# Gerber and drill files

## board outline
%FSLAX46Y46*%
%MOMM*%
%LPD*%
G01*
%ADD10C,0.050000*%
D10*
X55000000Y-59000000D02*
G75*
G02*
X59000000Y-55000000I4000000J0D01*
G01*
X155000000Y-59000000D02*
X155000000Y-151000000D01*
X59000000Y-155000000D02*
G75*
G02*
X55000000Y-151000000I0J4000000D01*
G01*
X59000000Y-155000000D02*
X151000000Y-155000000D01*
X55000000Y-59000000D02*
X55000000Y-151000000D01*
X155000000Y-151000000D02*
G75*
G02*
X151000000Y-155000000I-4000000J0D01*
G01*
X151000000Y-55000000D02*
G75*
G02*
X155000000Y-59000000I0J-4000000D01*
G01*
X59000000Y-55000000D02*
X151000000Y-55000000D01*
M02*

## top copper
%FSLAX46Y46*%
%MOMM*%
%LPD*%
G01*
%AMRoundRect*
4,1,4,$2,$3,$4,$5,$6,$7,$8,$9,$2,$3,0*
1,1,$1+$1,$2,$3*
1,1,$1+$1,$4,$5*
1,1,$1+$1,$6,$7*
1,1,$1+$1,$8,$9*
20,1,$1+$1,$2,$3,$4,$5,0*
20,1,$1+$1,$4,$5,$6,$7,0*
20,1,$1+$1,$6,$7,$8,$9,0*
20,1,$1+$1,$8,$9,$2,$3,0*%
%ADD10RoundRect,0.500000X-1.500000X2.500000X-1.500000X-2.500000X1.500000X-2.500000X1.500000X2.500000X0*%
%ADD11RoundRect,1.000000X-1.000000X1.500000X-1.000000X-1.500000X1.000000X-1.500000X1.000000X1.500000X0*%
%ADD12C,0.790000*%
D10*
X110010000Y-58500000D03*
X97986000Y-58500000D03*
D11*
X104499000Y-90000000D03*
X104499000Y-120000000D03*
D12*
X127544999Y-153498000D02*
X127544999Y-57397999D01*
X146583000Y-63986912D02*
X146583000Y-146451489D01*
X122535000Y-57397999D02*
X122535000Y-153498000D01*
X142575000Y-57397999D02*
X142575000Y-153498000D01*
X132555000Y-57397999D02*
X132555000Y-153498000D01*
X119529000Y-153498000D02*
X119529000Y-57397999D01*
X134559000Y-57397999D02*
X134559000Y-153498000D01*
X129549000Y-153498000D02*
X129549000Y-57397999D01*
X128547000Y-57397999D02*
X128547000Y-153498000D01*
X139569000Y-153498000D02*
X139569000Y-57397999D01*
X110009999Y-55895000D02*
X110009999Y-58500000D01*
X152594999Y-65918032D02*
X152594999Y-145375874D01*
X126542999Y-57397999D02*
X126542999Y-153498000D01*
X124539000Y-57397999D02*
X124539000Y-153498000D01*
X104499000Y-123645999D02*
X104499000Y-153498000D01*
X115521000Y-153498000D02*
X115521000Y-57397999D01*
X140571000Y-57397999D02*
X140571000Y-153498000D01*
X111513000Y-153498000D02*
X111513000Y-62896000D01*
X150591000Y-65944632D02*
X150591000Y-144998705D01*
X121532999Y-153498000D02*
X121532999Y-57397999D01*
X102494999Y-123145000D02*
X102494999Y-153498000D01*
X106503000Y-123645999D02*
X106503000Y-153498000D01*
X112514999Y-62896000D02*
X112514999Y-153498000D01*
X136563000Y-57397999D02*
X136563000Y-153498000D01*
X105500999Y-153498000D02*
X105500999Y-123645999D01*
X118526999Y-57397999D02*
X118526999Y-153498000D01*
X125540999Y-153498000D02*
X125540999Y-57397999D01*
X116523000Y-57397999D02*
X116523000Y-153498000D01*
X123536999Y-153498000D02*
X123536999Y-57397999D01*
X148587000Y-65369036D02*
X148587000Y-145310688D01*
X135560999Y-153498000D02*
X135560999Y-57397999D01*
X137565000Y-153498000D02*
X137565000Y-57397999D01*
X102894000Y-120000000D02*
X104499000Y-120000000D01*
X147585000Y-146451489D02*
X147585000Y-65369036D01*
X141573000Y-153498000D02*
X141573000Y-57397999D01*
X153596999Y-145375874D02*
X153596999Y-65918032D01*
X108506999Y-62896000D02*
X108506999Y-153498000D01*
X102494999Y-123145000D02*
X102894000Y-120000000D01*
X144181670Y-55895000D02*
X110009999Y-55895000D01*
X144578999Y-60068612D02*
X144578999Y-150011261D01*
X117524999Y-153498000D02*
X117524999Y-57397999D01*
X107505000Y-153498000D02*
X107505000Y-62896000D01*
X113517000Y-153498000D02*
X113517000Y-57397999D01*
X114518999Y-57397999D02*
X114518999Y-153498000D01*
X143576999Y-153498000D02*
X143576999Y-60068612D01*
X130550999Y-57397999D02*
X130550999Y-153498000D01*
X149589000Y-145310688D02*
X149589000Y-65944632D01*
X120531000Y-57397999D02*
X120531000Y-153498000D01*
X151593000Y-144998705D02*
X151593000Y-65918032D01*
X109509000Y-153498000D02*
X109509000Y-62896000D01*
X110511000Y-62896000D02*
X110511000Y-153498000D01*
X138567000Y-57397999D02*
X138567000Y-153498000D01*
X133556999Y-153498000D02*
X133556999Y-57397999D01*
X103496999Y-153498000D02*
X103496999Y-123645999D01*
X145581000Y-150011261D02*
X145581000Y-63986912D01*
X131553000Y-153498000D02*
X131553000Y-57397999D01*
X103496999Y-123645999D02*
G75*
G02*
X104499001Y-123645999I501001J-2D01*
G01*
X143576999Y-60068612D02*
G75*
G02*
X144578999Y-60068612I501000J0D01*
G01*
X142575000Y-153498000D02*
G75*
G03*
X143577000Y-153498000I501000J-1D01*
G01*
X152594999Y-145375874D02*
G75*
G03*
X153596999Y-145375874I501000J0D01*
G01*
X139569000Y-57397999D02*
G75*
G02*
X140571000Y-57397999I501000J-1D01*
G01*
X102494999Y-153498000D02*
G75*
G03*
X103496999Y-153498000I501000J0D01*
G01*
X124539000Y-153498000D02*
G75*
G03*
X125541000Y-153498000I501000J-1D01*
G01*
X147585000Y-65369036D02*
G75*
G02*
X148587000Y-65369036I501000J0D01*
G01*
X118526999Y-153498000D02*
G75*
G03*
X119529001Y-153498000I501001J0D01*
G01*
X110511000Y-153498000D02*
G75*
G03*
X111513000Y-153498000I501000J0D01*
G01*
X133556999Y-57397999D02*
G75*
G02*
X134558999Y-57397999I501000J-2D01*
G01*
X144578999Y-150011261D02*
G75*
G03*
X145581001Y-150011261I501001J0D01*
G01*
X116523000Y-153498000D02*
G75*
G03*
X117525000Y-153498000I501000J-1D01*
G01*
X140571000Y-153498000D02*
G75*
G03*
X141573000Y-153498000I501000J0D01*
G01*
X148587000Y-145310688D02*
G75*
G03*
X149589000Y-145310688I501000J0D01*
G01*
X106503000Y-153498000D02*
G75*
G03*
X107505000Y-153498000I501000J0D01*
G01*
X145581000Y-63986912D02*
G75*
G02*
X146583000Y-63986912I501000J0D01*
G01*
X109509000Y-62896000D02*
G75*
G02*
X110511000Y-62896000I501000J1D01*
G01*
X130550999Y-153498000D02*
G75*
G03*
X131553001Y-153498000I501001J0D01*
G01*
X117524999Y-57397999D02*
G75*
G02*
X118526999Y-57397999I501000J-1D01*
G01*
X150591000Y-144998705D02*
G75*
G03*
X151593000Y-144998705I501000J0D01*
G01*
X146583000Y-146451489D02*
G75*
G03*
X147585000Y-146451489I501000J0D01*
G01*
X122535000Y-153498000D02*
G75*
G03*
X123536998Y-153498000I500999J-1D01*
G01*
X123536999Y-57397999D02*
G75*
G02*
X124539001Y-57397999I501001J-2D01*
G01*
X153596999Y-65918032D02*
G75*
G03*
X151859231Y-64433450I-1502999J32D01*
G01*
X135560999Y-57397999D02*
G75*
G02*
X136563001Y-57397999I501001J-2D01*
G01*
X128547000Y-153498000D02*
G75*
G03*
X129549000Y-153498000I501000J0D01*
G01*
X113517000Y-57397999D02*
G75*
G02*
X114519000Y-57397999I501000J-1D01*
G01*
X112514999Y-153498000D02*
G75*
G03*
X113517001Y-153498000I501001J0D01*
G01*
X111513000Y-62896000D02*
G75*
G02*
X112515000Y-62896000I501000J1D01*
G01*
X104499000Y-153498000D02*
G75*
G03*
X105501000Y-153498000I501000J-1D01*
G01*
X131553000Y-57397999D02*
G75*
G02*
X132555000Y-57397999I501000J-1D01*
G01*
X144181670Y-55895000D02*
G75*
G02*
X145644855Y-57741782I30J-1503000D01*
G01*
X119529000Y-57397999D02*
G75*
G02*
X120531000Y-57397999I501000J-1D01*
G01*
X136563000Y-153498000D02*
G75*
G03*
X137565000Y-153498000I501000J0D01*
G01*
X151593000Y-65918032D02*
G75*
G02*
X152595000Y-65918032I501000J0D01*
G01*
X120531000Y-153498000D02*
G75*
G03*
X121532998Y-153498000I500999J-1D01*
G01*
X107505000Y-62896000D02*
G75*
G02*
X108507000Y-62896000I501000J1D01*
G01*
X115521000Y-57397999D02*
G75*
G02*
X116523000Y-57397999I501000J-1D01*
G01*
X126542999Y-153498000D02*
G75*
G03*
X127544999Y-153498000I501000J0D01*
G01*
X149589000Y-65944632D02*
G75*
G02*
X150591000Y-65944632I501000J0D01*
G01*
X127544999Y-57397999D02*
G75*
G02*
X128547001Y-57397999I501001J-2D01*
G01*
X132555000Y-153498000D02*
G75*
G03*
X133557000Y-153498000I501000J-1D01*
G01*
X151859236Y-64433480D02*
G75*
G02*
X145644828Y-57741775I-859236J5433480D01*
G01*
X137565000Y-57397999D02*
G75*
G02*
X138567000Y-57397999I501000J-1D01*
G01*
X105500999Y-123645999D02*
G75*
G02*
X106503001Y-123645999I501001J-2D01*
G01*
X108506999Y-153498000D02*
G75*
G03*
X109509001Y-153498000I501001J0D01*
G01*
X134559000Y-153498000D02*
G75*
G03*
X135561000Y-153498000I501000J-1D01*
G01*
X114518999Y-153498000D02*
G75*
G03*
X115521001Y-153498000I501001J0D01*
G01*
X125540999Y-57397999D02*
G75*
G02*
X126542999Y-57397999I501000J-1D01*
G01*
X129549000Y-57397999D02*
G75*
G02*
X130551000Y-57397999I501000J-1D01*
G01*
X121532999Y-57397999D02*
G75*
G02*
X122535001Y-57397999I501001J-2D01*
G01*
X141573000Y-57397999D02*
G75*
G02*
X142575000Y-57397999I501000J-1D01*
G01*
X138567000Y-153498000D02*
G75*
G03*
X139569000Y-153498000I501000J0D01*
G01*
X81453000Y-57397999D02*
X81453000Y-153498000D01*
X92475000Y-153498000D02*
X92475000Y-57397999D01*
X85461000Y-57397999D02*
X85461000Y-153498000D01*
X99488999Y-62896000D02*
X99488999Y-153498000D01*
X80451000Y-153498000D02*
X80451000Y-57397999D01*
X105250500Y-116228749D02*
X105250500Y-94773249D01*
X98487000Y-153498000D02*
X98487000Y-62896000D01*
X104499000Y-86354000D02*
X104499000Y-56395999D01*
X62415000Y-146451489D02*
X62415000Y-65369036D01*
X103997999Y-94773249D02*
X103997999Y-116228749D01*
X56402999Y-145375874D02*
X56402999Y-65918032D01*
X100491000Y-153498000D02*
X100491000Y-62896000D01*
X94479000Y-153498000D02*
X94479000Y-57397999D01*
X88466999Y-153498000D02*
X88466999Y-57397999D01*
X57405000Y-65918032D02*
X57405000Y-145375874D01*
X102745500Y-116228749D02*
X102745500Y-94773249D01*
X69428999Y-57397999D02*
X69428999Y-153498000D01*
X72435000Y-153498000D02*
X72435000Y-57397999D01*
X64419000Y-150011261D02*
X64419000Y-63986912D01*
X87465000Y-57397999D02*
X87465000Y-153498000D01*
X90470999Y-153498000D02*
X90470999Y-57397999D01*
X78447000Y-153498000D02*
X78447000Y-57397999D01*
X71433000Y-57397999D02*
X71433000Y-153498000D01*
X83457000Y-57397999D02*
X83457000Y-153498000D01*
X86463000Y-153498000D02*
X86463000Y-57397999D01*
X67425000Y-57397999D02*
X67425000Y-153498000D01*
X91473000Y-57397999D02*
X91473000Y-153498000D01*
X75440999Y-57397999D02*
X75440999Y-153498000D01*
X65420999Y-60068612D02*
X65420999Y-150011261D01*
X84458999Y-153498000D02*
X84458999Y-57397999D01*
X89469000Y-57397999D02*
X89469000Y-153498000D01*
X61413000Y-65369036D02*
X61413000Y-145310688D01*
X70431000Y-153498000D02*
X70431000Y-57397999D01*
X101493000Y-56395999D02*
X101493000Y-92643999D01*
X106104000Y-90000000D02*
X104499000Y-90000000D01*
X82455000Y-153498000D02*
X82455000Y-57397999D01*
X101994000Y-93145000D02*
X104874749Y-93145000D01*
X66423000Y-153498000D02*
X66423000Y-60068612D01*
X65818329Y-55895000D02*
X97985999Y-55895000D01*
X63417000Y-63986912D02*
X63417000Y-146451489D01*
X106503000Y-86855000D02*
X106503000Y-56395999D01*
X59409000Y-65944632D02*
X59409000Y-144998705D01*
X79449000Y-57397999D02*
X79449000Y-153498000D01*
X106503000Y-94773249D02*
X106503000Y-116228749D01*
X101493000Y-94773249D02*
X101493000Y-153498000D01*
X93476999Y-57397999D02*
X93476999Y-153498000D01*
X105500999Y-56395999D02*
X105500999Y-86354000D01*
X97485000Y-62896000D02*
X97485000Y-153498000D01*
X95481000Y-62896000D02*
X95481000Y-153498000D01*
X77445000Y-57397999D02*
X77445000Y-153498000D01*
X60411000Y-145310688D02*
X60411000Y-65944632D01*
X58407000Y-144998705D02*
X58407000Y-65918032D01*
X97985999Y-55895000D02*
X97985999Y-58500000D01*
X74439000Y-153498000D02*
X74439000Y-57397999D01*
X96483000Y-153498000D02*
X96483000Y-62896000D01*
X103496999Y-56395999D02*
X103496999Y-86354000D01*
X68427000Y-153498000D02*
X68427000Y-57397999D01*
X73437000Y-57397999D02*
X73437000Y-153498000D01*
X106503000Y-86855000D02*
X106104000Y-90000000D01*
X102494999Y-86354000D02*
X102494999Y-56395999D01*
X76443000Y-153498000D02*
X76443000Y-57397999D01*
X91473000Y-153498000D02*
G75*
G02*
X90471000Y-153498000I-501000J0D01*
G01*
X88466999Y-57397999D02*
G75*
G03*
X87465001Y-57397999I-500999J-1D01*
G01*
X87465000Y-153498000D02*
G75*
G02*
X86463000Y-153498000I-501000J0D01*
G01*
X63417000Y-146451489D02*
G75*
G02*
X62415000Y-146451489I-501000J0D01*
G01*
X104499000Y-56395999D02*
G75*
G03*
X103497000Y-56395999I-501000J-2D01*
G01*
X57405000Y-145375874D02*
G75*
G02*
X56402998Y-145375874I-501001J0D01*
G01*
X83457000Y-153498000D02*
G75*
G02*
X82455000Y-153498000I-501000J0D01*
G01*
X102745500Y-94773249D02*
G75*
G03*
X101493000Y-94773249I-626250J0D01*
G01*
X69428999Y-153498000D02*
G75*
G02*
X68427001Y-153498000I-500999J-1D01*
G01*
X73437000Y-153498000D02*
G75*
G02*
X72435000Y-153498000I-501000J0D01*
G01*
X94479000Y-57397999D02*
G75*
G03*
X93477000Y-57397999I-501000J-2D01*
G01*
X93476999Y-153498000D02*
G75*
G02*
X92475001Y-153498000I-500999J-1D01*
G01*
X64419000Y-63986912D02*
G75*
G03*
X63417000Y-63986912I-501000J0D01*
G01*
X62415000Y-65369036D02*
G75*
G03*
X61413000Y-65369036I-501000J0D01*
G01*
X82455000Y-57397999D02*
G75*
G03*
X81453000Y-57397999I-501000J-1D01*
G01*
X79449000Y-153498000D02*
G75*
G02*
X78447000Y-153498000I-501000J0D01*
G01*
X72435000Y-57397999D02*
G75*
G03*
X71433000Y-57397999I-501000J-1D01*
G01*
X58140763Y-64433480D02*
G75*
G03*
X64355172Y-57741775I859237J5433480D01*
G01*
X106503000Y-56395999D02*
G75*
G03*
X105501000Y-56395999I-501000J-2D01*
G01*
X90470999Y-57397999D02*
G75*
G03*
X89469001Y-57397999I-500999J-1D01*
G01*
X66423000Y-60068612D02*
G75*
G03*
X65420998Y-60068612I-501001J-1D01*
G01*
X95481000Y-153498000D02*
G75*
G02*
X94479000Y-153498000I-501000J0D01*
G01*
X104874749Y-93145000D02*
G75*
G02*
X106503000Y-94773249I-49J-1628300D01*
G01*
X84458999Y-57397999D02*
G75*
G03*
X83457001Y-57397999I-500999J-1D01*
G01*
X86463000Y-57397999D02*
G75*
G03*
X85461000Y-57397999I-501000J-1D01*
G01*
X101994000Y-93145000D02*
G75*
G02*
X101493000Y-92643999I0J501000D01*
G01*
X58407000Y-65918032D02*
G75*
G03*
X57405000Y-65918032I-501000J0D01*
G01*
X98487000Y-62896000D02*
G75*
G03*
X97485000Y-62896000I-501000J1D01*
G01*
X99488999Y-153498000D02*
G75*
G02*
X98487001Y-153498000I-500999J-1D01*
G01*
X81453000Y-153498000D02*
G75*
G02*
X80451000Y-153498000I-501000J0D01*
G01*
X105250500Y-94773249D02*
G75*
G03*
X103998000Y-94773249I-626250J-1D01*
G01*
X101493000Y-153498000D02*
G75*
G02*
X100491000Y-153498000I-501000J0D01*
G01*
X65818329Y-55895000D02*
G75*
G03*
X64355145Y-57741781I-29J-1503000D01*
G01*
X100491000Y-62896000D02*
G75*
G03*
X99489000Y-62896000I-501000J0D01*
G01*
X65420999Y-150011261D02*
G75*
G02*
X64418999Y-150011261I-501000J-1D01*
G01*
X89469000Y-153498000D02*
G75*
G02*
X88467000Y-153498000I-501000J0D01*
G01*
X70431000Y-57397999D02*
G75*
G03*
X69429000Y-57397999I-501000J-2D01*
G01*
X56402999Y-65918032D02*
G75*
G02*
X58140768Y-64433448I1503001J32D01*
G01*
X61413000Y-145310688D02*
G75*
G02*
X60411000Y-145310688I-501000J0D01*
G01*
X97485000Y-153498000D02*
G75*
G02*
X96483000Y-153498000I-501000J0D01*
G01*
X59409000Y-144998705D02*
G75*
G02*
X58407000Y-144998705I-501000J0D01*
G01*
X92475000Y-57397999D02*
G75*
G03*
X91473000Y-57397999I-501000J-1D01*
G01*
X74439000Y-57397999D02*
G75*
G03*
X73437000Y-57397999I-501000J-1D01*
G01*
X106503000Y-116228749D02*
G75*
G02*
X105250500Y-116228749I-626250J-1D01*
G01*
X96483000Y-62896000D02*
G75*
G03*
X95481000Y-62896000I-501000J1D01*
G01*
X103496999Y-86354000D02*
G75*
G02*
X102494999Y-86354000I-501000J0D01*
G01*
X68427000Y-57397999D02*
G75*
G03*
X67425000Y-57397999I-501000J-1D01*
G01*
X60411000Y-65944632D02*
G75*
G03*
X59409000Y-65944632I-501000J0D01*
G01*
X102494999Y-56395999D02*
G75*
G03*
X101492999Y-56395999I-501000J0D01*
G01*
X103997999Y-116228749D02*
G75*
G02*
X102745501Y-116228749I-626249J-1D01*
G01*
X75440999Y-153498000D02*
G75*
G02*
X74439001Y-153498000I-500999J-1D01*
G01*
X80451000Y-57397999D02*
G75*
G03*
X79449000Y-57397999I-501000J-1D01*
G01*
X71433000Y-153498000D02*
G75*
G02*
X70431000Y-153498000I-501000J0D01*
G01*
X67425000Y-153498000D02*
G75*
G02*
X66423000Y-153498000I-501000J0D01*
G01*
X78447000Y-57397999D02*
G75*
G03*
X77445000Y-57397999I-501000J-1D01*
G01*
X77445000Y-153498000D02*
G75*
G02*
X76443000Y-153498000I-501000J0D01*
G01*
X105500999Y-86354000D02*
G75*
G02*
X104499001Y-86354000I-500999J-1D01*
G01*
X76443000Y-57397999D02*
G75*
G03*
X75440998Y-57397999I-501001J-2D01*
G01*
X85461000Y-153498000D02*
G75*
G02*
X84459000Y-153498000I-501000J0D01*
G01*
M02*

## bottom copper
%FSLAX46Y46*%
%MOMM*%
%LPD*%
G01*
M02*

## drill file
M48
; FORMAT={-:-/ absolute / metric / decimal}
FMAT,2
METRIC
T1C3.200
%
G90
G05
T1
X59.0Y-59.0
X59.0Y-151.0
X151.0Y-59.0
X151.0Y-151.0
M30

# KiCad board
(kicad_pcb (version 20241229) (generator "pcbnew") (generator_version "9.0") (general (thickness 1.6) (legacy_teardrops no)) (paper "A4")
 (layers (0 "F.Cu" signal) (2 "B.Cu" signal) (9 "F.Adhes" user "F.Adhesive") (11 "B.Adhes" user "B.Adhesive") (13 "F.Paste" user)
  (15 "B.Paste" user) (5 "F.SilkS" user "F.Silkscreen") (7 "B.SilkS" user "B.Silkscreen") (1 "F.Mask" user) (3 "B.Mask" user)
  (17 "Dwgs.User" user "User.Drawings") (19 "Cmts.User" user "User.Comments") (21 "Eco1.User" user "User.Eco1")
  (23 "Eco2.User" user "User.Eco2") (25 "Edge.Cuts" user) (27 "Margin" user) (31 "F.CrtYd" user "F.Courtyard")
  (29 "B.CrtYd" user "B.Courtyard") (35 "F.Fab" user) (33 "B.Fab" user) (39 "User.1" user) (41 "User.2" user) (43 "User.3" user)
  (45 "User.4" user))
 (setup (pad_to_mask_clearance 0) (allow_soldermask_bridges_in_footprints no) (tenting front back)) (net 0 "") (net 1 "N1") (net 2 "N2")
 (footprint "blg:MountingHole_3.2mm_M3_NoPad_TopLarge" (layer "F.Cu") (at 151 59)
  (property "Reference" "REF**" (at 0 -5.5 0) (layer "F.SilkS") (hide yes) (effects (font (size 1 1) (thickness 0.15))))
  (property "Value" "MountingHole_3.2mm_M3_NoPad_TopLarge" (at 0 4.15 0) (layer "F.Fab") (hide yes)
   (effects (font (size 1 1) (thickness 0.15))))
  (pad "" np_thru_hole circle (at 0 0) (size 7.6 7.6) (drill 3.2) (layers) (zone_connect 2)))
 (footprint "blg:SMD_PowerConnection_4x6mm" (layer "F.Cu") (at 110.01 58.5 -90)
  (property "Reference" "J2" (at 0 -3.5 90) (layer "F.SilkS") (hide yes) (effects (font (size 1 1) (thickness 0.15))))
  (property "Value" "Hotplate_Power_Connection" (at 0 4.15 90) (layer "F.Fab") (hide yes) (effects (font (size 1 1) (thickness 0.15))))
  (pad "1" smd roundrect (at 0 0 270) (size 6 4) (layers "F.Cu" "F.Mask" "F.Paste") (roundrect_rratio 0.125) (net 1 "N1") (zone_connect 2)))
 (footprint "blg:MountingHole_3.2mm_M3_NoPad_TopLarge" (layer "F.Cu") (at 59 151)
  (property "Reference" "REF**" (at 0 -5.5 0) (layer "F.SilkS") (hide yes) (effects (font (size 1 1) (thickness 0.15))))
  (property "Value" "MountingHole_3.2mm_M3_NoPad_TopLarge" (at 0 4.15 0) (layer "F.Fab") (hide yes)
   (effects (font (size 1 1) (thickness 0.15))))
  (pad "" np_thru_hole circle (at 0 0) (size 7.6 7.6) (drill 3.2) (layers) (zone_connect 2)))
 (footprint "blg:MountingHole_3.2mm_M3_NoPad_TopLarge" (layer "F.Cu") (at 151 151)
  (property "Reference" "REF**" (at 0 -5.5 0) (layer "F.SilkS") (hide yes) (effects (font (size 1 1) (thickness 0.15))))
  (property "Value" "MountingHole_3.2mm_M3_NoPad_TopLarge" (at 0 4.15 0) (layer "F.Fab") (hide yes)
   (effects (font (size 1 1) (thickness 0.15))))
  (pad "" np_thru_hole circle (at 0 0) (size 7.6 7.6) (drill 3.2) (layers) (zone_connect 2)))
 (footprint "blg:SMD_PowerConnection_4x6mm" (layer "F.Cu") (at 97.986 58.5 -90)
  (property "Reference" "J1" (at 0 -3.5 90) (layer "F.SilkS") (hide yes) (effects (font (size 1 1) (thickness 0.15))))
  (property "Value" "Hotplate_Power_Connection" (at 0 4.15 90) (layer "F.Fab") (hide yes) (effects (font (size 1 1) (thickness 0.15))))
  (pad "1" smd roundrect (at 0 0 270) (size 6 4) (layers "F.Cu" "F.Mask" "F.Paste") (roundrect_rratio 0.125) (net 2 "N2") (zone_connect 2)))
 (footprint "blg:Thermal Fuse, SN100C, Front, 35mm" (layer "F.Cu") (at 104.499 105 -90)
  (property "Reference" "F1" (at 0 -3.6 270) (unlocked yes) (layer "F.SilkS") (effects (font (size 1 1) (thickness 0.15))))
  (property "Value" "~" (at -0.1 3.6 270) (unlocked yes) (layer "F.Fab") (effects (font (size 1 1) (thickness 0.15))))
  (pad "1" smd roundrect (at -15 0 270) (size 5 4) (layers "F.Cu" "F.Mask") (roundrect_rratio 0.25) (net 2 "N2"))
  (pad "2" smd roundrect (at 15 0 270) (size 5 4) (layers "F.Cu" "F.Mask") (roundrect_rratio 0.25) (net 1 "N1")))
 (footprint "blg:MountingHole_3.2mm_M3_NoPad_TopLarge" (layer "F.Cu") (at 59 59)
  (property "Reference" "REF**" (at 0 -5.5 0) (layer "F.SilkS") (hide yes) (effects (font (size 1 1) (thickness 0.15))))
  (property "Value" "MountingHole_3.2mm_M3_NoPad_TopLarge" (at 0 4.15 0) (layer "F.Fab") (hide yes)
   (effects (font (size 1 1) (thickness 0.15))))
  (pad "" np_thru_hole circle (at 0 0) (size 7.6 7.6) (drill 3.2) (layers) (zone_connect 2)))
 (gr_arc (start 55 59) (mid 56.171573 56.171573) (end 59 55) (stroke (width 0.05) (type solid)) (layer "Edge.Cuts"))
 (gr_line (start 155 59) (end 155 151) (stroke (width 0.05) (type default)) (layer "Edge.Cuts"))
 (gr_arc (start 59 155) (mid 56.171573 153.828427) (end 55 151) (stroke (width 0.05) (type solid)) (layer "Edge.Cuts"))
 (gr_line (start 59 155) (end 151 155) (stroke (width 0.05) (type default)) (layer "Edge.Cuts"))
 (gr_line (start 55 59) (end 55 151) (stroke (width 0.05) (type default)) (layer "Edge.Cuts"))
 (gr_arc (start 155 151) (mid 153.828427 153.828427) (end 151 155) (stroke (width 0.05) (type solid)) (layer "Edge.Cuts"))
 (gr_arc (start 151 55) (mid 153.828427 56.171573) (end 155 59) (stroke (width 0.05) (type solid)) (layer "Edge.Cuts"))
 (gr_line (start 59 55) (end 151 55) (stroke (width 0.05) (type default)) (layer "Edge.Cuts"))
 (segment (start 127.544999 153.498) (end 127.544999 57.397999) (width 0.79) (layer "F.Cu") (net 1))
 (segment (start 146.583 63.986912) (end 146.583 146.451489) (width 0.79) (layer "F.Cu") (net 1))
 (segment (start 122.535 57.397999) (end 122.535 153.498) (width 0.79) (layer "F.Cu") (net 1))
 (segment (start 142.575 57.397999) (end 142.575 153.498) (width 0.79) (layer "F.Cu") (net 1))
 (segment (start 132.555 57.397999) (end 132.555 153.498) (width 0.79) (layer "F.Cu") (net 1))
 (segment (start 119.529 153.498) (end 119.529 57.397999) (width 0.79) (layer "F.Cu") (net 1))
 (segment (start 134.559 57.397999) (end 134.559 153.498) (width 0.79) (layer "F.Cu") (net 1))
 (segment (start 129.549 153.498) (end 129.549 57.397999) (width 0.79) (layer "F.Cu") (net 1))
 (segment (start 128.547 57.397999) (end 128.547 153.498) (width 0.79) (layer "F.Cu") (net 1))
 (segment (start 139.569 153.498) (end 139.569 57.397999) (width 0.79) (layer "F.Cu") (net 1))
 (segment (start 110.009999 55.895) (end 110.009999 58.5) (width 0.79) (layer "F.Cu") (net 1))
 (segment (start 152.594999 65.918032) (end 152.594999 145.375874) (width 0.79) (layer "F.Cu") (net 1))
 (segment (start 126.542999 57.397999) (end 126.542999 153.498) (width 0.79) (layer "F.Cu") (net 1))
 (segment (start 124.539 57.397999) (end 124.539 153.498) (width 0.79) (layer "F.Cu") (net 1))
 (segment (start 104.499 123.645999) (end 104.499 153.498) (width 0.79) (layer "F.Cu") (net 1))
 (segment (start 115.521 153.498) (end 115.521 57.397999) (width 0.79) (layer "F.Cu") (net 1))
 (segment (start 140.571 57.397999) (end 140.571 153.498) (width 0.79) (layer "F.Cu") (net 1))
 (segment (start 111.513 153.498) (end 111.513 62.896) (width 0.79) (layer "F.Cu") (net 1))
 (segment (start 150.591 65.944632) (end 150.591 144.998705) (width 0.79) (layer "F.Cu") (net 1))
 (segment (start 121.532999 153.498) (end 121.532999 57.397999) (width 0.79) (layer "F.Cu") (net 1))
 (segment (start 102.494999 123.145) (end 102.494999 153.498) (width 0.79) (layer "F.Cu") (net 1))
 (segment (start 106.503 123.645999) (end 106.503 153.498) (width 0.79) (layer "F.Cu") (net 1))
 (segment (start 112.514999 62.896) (end 112.514999 153.498) (width 0.79) (layer "F.Cu") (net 1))
 (segment (start 136.563 57.397999) (end 136.563 153.498) (width 0.79) (layer "F.Cu") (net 1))
 (segment (start 105.500999 153.498) (end 105.500999 123.645999) (width 0.79) (layer "F.Cu") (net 1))
 (segment (start 118.526999 57.397999) (end 118.526999 153.498) (width 0.79) (layer "F.Cu") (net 1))
 (segment (start 125.540999 153.498) (end 125.540999 57.397999) (width 0.79) (layer "F.Cu") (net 1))
 (segment (start 116.523 57.397999) (end 116.523 153.498) (width 0.79) (layer "F.Cu") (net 1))
 (segment (start 123.536999 153.498) (end 123.536999 57.397999) (width 0.79) (layer "F.Cu") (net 1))
 (segment (start 148.587 65.369036) (end 148.587 145.310688) (width 0.79) (layer "F.Cu") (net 1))
 (segment (start 135.560999 153.498) (end 135.560999 57.397999) (width 0.79) (layer "F.Cu") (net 1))
 (segment (start 137.565 153.498) (end 137.565 57.397999) (width 0.79) (layer "F.Cu") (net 1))
 (segment (start 102.894 120) (end 104.499 120) (width 0.79) (layer "F.Cu") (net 1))
 (segment (start 147.585 146.451489) (end 147.585 65.369036) (width 0.79) (layer "F.Cu") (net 1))
 (segment (start 141.573 153.498) (end 141.573 57.397999) (width 0.79) (layer "F.Cu") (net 1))
 (segment (start 153.596999 145.375874) (end 153.596999 65.918032) (width 0.79) (layer "F.Cu") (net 1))
 (segment (start 108.506999 62.896) (end 108.506999 153.498) (width 0.79) (layer "F.Cu") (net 1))
 (segment (start 102.494999 123.145) (end 102.894 120) (width 0.79) (layer "F.Cu") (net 1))
 (segment (start 144.18167 55.895) (end 110.009999 55.895) (width 0.79) (layer "F.Cu") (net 1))
 (segment (start 144.578999 60.068612) (end 144.578999 150.011261) (width 0.79) (layer "F.Cu") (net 1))
 (segment (start 117.524999 153.498) (end 117.524999 57.397999) (width 0.79) (layer "F.Cu") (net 1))
 (segment (start 107.505 153.498) (end 107.505 62.896) (width 0.79) (layer "F.Cu") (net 1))
 (segment (start 113.517 153.498) (end 113.517 57.397999) (width 0.79) (layer "F.Cu") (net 1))
 (segment (start 114.518999 57.397999) (end 114.518999 153.498) (width 0.79) (layer "F.Cu") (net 1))
 (segment (start 143.576999 153.498) (end 143.576999 60.068612) (width 0.79) (layer "F.Cu") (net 1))
 (segment (start 130.550999 57.397999) (end 130.550999 153.498) (width 0.79) (layer "F.Cu") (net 1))
 (segment (start 149.589 145.310688) (end 149.589 65.944632) (width 0.79) (layer "F.Cu") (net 1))
 (segment (start 120.531 57.397999) (end 120.531 153.498) (width 0.79) (layer "F.Cu") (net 1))
 (segment (start 151.593 144.998705) (end 151.593 65.918032) (width 0.79) (layer "F.Cu") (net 1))
 (segment (start 109.509 153.498) (end 109.509 62.896) (width 0.79) (layer "F.Cu") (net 1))
 (segment (start 110.511 62.896) (end 110.511 153.498) (width 0.79) (layer "F.Cu") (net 1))
 (segment (start 138.567 57.397999) (end 138.567 153.498) (width 0.79) (layer "F.Cu") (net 1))
 (segment (start 133.556999 153.498) (end 133.556999 57.397999) (width 0.79) (layer "F.Cu") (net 1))
 (segment (start 103.496999 153.498) (end 103.496999 123.645999) (width 0.79) (layer "F.Cu") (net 1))
 (segment (start 145.581 150.011261) (end 145.581 63.986912) (width 0.79) (layer "F.Cu") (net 1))
 (segment (start 131.553 153.498) (end 131.553 57.397999) (width 0.79) (layer "F.Cu") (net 1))
 (arc (start 103.496999 123.645999) (mid 103.997999 123.145) (end 104.499 123.645999) (width 0.79) (layer "F.Cu") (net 1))
 (arc (start 143.576999 60.068612) (mid 144.077999 59.567612) (end 144.578999 60.068612) (width 0.79) (layer "F.Cu") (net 1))
 (arc (start 142.575 153.498) (mid 143.076 153.999) (end 143.576999 153.498) (width 0.79) (layer "F.Cu") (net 1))
 (arc (start 152.594999 145.375874) (mid 153.095999 145.876874) (end 153.596999 145.375874) (width 0.79) (layer "F.Cu") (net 1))
 (arc (start 139.569 57.397999) (mid 140.07 56.897) (end 140.571 57.397999) (width 0.79) (layer "F.Cu") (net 1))
 (arc (start 102.494999 153.498) (mid 102.996 153.999) (end 103.496999 153.498) (width 0.79) (layer "F.Cu") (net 1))
 (arc (start 124.539 153.498) (mid 125.039999 153.999) (end 125.540999 153.498) (width 0.79) (layer "F.Cu") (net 1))
 (arc (start 147.585 65.369036) (mid 148.085999 64.868036) (end 148.587 65.369036) (width 0.79) (layer "F.Cu") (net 1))
 (arc (start 118.526999 153.498) (mid 119.027999 153.999) (end 119.529 153.498) (width 0.79) (layer "F.Cu") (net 1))
 (arc (start 110.511 153.498) (mid 111.012 153.999) (end 111.513 153.498) (width 0.79) (layer "F.Cu") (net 1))
 (arc (start 133.556999 57.397999) (mid 134.058 56.897) (end 134.559 57.397999) (width 0.79) (layer "F.Cu") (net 1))
 (arc (start 144.578999 150.011261) (mid 145.079999 150.512261) (end 145.581 150.011261) (width 0.79) (layer "F.Cu") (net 1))
 (arc (start 116.523 153.498) (mid 117.023999 153.999) (end 117.524999 153.498) (width 0.79) (layer "F.Cu") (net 1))
 (arc (start 140.571 153.498) (mid 141.072 153.999) (end 141.573 153.498) (width 0.79) (layer "F.Cu") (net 1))
 (arc (start 148.587 145.310688) (mid 149.088 145.811688) (end 149.589 145.310688) (width 0.79) (layer "F.Cu") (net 1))
 (arc (start 106.503 153.498) (mid 107.004 153.999) (end 107.505 153.498) (width 0.79) (layer "F.Cu") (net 1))
 (arc (start 145.581 63.986912) (mid 146.082 63.485912) (end 146.583 63.986912) (width 0.79) (layer "F.Cu") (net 1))
 (arc (start 109.509 62.896) (mid 110.009999 62.394999) (end 110.511 62.896) (width 0.79) (layer "F.Cu") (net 1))
 (arc (start 130.550999 153.498) (mid 131.051999 153.999) (end 131.553 153.498) (width 0.79) (layer "F.Cu") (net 1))
 (arc (start 117.524999 57.397999) (mid 118.026 56.897) (end 118.526999 57.397999) (width 0.79) (layer "F.Cu") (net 1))
 (arc (start 150.591 144.998705) (mid 151.092 145.499705) (end 151.593 144.998705) (width 0.79) (layer "F.Cu") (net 1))
 (arc (start 146.583 146.451489) (mid 147.084 146.952489) (end 147.585 146.451489) (width 0.79) (layer "F.Cu") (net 1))
 (arc (start 122.535 153.498) (mid 123.035999 153.999) (end 123.536999 153.498) (width 0.79) (layer "F.Cu") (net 1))
 (arc (start 123.536999 57.397999) (mid 124.038 56.897) (end 124.539 57.397999) (width 0.79) (layer "F.Cu") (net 1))
 (arc (start 153.596999 65.918032) (mid 153.21163 64.91309) (end 151.859236 64.43348) (width 0.79) (layer "F.Cu") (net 1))
 (arc (start 135.560999 57.397999) (mid 136.061999 56.897) (end 136.563 57.397999) (width 0.79) (layer "F.Cu") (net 1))
 (arc (start 128.547 153.498) (mid 129.048 153.999) (end 129.549 153.498) (width 0.79) (layer "F.Cu") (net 1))
 (arc (start 113.517 57.397999) (mid 114.018 56.897) (end 114.518999 57.397999) (width 0.79) (layer "F.Cu") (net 1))
 (arc (start 112.514999 153.498) (mid 113.015999 153.999) (end 113.517 153.498) (width 0.79) (layer "F.Cu") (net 1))
 (arc (start 111.513 62.896) (mid 112.013999 62.394999) (end 112.514999 62.896) (width 0.79) (layer "F.Cu") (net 1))
 (arc (start 104.499 153.498) (mid 105 153.999) (end 105.500999 153.498) (width 0.79) (layer "F.Cu") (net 1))
 (arc (start 131.553 57.397999) (mid 132.054 56.897) (end 132.555 57.397999) (width 0.79) (layer "F.Cu") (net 1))
 (arc (start 144.18167 55.895) (mid 145.359742 56.464642) (end 145.644827 57.741775) (width 0.79) (layer "F.Cu") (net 1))
 (arc (start 119.529 57.397999) (mid 120.03 56.897) (end 120.531 57.397999) (width 0.79) (layer "F.Cu") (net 1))
 (arc (start 136.563 153.498) (mid 137.064 153.999) (end 137.565 153.498) (width 0.79) (layer "F.Cu") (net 1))
 (arc (start 151.593 65.918032) (mid 152.094 65.417032) (end 152.594999 65.918032) (width 0.79) (layer "F.Cu") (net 1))
 (arc (start 120.531 153.498) (mid 121.032 153.999) (end 121.532999 153.498) (width 0.79) (layer "F.Cu") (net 1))
 (arc (start 107.505 62.896) (mid 108.005999 62.394999) (end 108.506999 62.896) (width 0.79) (layer "F.Cu") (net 1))
 (arc (start 115.521 57.397999) (mid 116.022 56.897) (end 116.523 57.397999) (width 0.79) (layer "F.Cu") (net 1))
 (arc (start 126.542999 153.498) (mid 127.044 153.999) (end 127.544999 153.498) (width 0.79) (layer "F.Cu") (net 1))
 (arc (start 149.589 65.944632) (mid 150.09 65.443632) (end 150.591 65.944632) (width 0.79) (layer "F.Cu") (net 1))
 (arc (start 127.544999 57.397999) (mid 128.045999 56.897) (end 128.547 57.397999) (width 0.79) (layer "F.Cu") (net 1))
 (arc (start 132.555 153.498) (mid 133.056 153.999) (end 133.556999 153.498) (width 0.79) (layer "F.Cu") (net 1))
 (arc (start 151.859236 64.43348) (mid 146.969108 62.743382) (end 145.644827 57.741775) (width 0.79) (layer "F.Cu") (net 1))
 (arc (start 137.565 57.397999) (mid 138.066 56.897) (end 138.567 57.397999) (width 0.79) (layer "F.Cu") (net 1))
 (arc (start 105.500999 123.645999) (mid 106.002 123.145) (end 106.503 123.645999) (width 0.79) (layer "F.Cu") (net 1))
 (arc (start 108.506999 153.498) (mid 109.008 153.999) (end 109.509 153.498) (width 0.79) (layer "F.Cu") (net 1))
 (arc (start 134.559 153.498) (mid 135.059999 153.999) (end 135.560999 153.498) (width 0.79) (layer "F.Cu") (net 1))
 (arc (start 114.518999 153.498) (mid 115.02 153.999) (end 115.521 153.498) (width 0.79) (layer "F.Cu") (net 1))
 (arc (start 125.540999 57.397999) (mid 126.041999 56.897) (end 126.542999 57.397999) (width 0.79) (layer "F.Cu") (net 1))
 (arc (start 129.549 57.397999) (mid 130.05 56.897) (end 130.550999 57.397999) (width 0.79) (layer "F.Cu") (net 1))
 (arc (start 121.532999 57.397999) (mid 122.033999 56.897) (end 122.535 57.397999) (width 0.79) (layer "F.Cu") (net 1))
 (arc (start 141.573 57.397999) (mid 142.074 56.897) (end 142.575 57.397999) (width 0.79) (layer "F.Cu") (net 1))
 (arc (start 138.567 153.498) (mid 139.067999 153.999) (end 139.569 153.498) (width 0.79) (layer "F.Cu") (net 1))
 (segment (start 81.453 57.397999) (end 81.453 153.498) (width 0.79) (layer "F.Cu") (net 2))
 (segment (start 92.475 153.498) (end 92.475 57.397999) (width 0.79) (layer "F.Cu") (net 2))
 (segment (start 85.461 57.397999) (end 85.461 153.498) (width 0.79) (layer "F.Cu") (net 2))
 (segment (start 99.488999 62.896) (end 99.488999 153.498) (width 0.79) (layer "F.Cu") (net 2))
 (segment (start 80.451 153.498) (end 80.451 57.397999) (width 0.79) (layer "F.Cu") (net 2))
 (segment (start 105.2505 116.228749) (end 105.2505 94.773249) (width 0.79) (layer "F.Cu") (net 2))
 (segment (start 98.487 153.498) (end 98.487 62.896) (width 0.79) (layer "F.Cu") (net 2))
 (segment (start 104.499 86.354) (end 104.499 56.395999) (width 0.79) (layer "F.Cu") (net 2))
 (segment (start 62.415 146.451489) (end 62.415 65.369036) (width 0.79) (layer "F.Cu") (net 2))
 (segment (start 103.997999 94.773249) (end 103.997999 116.228749) (width 0.79) (layer "F.Cu") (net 2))
 (segment (start 56.402999 145.375874) (end 56.402999 65.918032) (width 0.79) (layer "F.Cu") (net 2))
 (segment (start 100.491 153.498) (end 100.491 62.896) (width 0.79) (layer "F.Cu") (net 2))
 (segment (start 94.479 153.498) (end 94.479 57.397999) (width 0.79) (layer "F.Cu") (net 2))
 (segment (start 88.466999 153.498) (end 88.466999 57.397999) (width 0.79) (layer "F.Cu") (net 2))
 (segment (start 57.405 65.918032) (end 57.405 145.375874) (width 0.79) (layer "F.Cu") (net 2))
 (segment (start 102.7455 116.228749) (end 102.7455 94.773249) (width 0.79) (layer "F.Cu") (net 2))
 (segment (start 69.428999 57.397999) (end 69.428999 153.498) (width 0.79) (layer "F.Cu") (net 2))
 (segment (start 72.435 153.498) (end 72.435 57.397999) (width 0.79) (layer "F.Cu") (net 2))
 (segment (start 64.419 150.011261) (end 64.419 63.986912) (width 0.79) (layer "F.Cu") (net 2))
 (segment (start 87.465 57.397999) (end 87.465 153.498) (width 0.79) (layer "F.Cu") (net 2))
 (segment (start 90.470999 153.498) (end 90.470999 57.397999) (width 0.79) (layer "F.Cu") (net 2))
 (segment (start 78.447 153.498) (end 78.447 57.397999) (width 0.79) (layer "F.Cu") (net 2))
 (segment (start 71.433 57.397999) (end 71.433 153.498) (width 0.79) (layer "F.Cu") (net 2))
 (segment (start 83.457 57.397999) (end 83.457 153.498) (width 0.79) (layer "F.Cu") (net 2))
 (segment (start 86.463 153.498) (end 86.463 57.397999) (width 0.79) (layer "F.Cu") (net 2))
 (segment (start 67.425 57.397999) (end 67.425 153.498) (width 0.79) (layer "F.Cu") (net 2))
 (segment (start 91.473 57.397999) (end 91.473 153.498) (width 0.79) (layer "F.Cu") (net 2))
 (segment (start 75.440999 57.397999) (end 75.440999 153.498) (width 0.79) (layer "F.Cu") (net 2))
 (segment (start 65.420999 60.068612) (end 65.420999 150.011261) (width 0.79) (layer "F.Cu") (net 2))
 (segment (start 84.458999 153.498) (end 84.458999 57.397999) (width 0.79) (layer "F.Cu") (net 2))
 (segment (start 89.469 57.397999) (end 89.469 153.498) (width 0.79) (layer "F.Cu") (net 2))
 (segment (start 61.413 65.369036) (end 61.413 145.310688) (width 0.79) (layer "F.Cu") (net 2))
 (segment (start 70.431 153.498) (end 70.431 57.397999) (width 0.79) (layer "F.Cu") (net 2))
 (segment (start 101.493 56.395999) (end 101.493 92.643999) (width 0.79) (layer "F.Cu") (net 2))
 (segment (start 106.104 90) (end 104.499 90) (width 0.79) (layer "F.Cu") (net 2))
 (segment (start 82.455 153.498) (end 82.455 57.397999) (width 0.79) (layer "F.Cu") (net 2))
 (segment (start 101.994 93.145) (end 104.874749 93.145) (width 0.79) (layer "F.Cu") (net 2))
 (segment (start 66.423 153.498) (end 66.423 60.068612) (width 0.79) (layer "F.Cu") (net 2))
 (segment (start 65.818329 55.895) (end 97.985999 55.895) (width 0.79) (layer "F.Cu") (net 2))
 (segment (start 63.417 63.986912) (end 63.417 146.451489) (width 0.79) (layer "F.Cu") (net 2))
 (segment (start 106.503 86.855) (end 106.503 56.395999) (width 0.79) (layer "F.Cu") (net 2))
 (segment (start 59.409 65.944632) (end 59.409 144.998705) (width 0.79) (layer "F.Cu") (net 2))
 (segment (start 79.449 57.397999) (end 79.449 153.498) (width 0.79) (layer "F.Cu") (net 2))
 (segment (start 106.503 94.773249) (end 106.503 116.228749) (width 0.79) (layer "F.Cu") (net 2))
 (segment (start 101.493 94.773249) (end 101.493 153.498) (width 0.79) (layer "F.Cu") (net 2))
 (segment (start 93.476999 57.397999) (end 93.476999 153.498) (width 0.79) (layer "F.Cu") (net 2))
 (segment (start 105.500999 56.395999) (end 105.500999 86.354) (width 0.79) (layer "F.Cu") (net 2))
 (segment (start 97.485 62.896) (end 97.485 153.498) (width 0.79) (layer "F.Cu") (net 2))
 (segment (start 95.481 62.896) (end 95.481 153.498) (width 0.79) (layer "F.Cu") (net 2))
 (segment (start 77.445 57.397999) (end 77.445 153.498) (width 0.79) (layer "F.Cu") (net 2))
 (segment (start 60.411 145.310688) (end 60.411 65.944632) (width 0.79) (layer "F.Cu") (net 2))
 (segment (start 58.407 144.998705) (end 58.407 65.918032) (width 0.79) (layer "F.Cu") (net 2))
 (segment (start 97.985999 55.895) (end 97.985999 58.5) (width 0.79) (layer "F.Cu") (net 2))
 (segment (start 74.439 153.498) (end 74.439 57.397999) (width 0.79) (layer "F.Cu") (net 2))
 (segment (start 96.483 153.498) (end 96.483 62.896) (width 0.79) (layer "F.Cu") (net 2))
 (segment (start 103.496999 56.395999) (end 103.496999 86.354) (width 0.79) (layer "F.Cu") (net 2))
 (segment (start 68.427 153.498) (end 68.427 57.397999) (width 0.79) (layer "F.Cu") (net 2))
 (segment (start 73.437 57.397999) (end 73.437 153.498) (width 0.79) (layer "F.Cu") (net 2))
 (segment (start 106.503 86.855) (end 106.104 90) (width 0.79) (layer "F.Cu") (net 2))
 (segment (start 102.494999 86.354) (end 102.494999 56.395999) (width 0.79) (layer "F.Cu") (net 2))
 (segment (start 76.443 153.498) (end 76.443 57.397999) (width 0.79) (layer "F.Cu") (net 2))
 (arc (start 91.473 153.498) (mid 90.972 153.999) (end 90.470999 153.498) (width 0.79) (layer "F.Cu") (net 2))
 (arc (start 88.466999 57.397999) (mid 87.966 56.897) (end 87.465 57.397999) (width 0.79) (layer "F.Cu") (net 2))
 (arc (start 87.465 153.498) (mid 86.964 153.999) (end 86.463 153.498) (width 0.79) (layer "F.Cu") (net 2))
 (arc (start 63.417 146.451489) (mid 62.916 146.952489) (end 62.415 146.451489) (width 0.79) (layer "F.Cu") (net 2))
 (arc (start 104.499 56.395999) (mid 103.997999 55.895) (end 103.496999 56.395999) (width 0.79) (layer "F.Cu") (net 2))
 (arc (start 57.405 145.375874) (mid 56.904 145.876874) (end 56.402999 145.375874) (width 0.79) (layer "F.Cu") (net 2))
 (arc (start 83.457 153.498) (mid 82.956 153.999) (end 82.455 153.498) (width 0.79) (layer "F.Cu") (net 2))
 (arc (start 102.7455 94.773249) (mid 102.11925 94.146999) (end 101.493 94.773249) (width 0.79) (layer "F.Cu") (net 2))
 (arc (start 69.428999 153.498) (mid 68.928 153.999) (end 68.427 153.498) (width 0.79) (layer "F.Cu") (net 2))
 (arc (start 73.437 153.498) (mid 72.936 153.999) (end 72.435 153.498) (width 0.79) (layer "F.Cu") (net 2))
 (arc (start 94.479 57.397999) (mid 93.978 56.897) (end 93.476999 57.397999) (width 0.79) (layer "F.Cu") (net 2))
 (arc (start 93.476999 153.498) (mid 92.975999 153.999) (end 92.475 153.498) (width 0.79) (layer "F.Cu") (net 2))
 (arc (start 64.419 63.986912) (mid 63.918 63.485912) (end 63.417 63.986912) (width 0.79) (layer "F.Cu") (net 2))
 (arc (start 62.415 65.369036) (mid 61.913999 64.868036) (end 61.413 65.369036) (width 0.79) (layer "F.Cu") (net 2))
 (arc (start 82.455 57.397999) (mid 81.954 56.897) (end 81.453 57.397999) (width 0.79) (layer "F.Cu") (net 2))
 (arc (start 79.449 153.498) (mid 78.948 153.999) (end 78.447 153.498) (width 0.79) (layer "F.Cu") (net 2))
 (arc (start 72.435 57.397999) (mid 71.934 56.897) (end 71.433 57.397999) (width 0.79) (layer "F.Cu") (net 2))
 (arc (start 58.140763 64.43348) (mid 63.030891 62.743382) (end 64.355172 57.741775) (width 0.79) (layer "F.Cu") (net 2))
 (arc (start 106.503 56.395999) (mid 106.002 55.895) (end 105.500999 56.395999) (width 0.79) (layer "F.Cu") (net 2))
 (arc (start 90.470999 57.397999) (mid 89.97 56.897) (end 89.469 57.397999) (width 0.79) (layer "F.Cu") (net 2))
 (arc (start 66.423 60.068612) (mid 65.922 59.567612) (end 65.420999 60.068612) (width 0.79) (layer "F.Cu") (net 2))
 (arc (start 95.481 153.498) (mid 94.979999 153.999) (end 94.479 153.498) (width 0.79) (layer "F.Cu") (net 2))
 (arc (start 104.874749 93.145) (mid 106.026096 93.621903) (end 106.503 94.773249) (width 0.79) (layer "F.Cu") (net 2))
 (arc (start 84.458999 57.397999) (mid 83.957999 56.897) (end 83.457 57.397999) (width 0.79) (layer "F.Cu") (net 2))
 (arc (start 86.463 57.397999) (mid 85.962 56.897) (end 85.461 57.397999) (width 0.79) (layer "F.Cu") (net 2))
 (arc (start 101.994 93.145) (mid 101.639739 92.99826) (end 101.493 92.643999) (width 0.79) (layer "F.Cu") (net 2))
 (arc (start 58.407 65.918032) (mid 57.906 65.417032) (end 57.405 65.918032) (width 0.79) (layer "F.Cu") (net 2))
 (arc (start 98.487 62.896) (mid 97.985999 62.394999) (end 97.485 62.896) (width 0.79) (layer "F.Cu") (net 2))
 (arc (start 99.488999 153.498) (mid 98.988 153.999) (end 98.487 153.498) (width 0.79) (layer "F.Cu") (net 2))
 (arc (start 81.453 153.498) (mid 80.952 153.999) (end 80.451 153.498) (width 0.79) (layer "F.Cu") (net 2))
 (arc (start 105.2505 94.773249) (mid 104.62425 94.146999) (end 103.997999 94.773249) (width 0.79) (layer "F.Cu") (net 2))
 (arc (start 101.493 153.498) (mid 100.992 153.999) (end 100.491 153.498) (width 0.79) (layer "F.Cu") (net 2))
 (arc (start 65.818329 55.895) (mid 64.640257 56.464642) (end 64.355172 57.741775) (width 0.79) (layer "F.Cu") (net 2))
 (arc (start 100.491 62.896) (mid 99.99 62.394999) (end 99.488999 62.896) (width 0.79) (layer "F.Cu") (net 2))
 (arc (start 65.420999 150.011261) (mid 64.919999 150.512261) (end 64.419 150.011261) (width 0.79) (layer "F.Cu") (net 2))
 (arc (start 89.469 153.498) (mid 88.967999 153.999) (end 88.466999 153.498) (width 0.79) (layer "F.Cu") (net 2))
 (arc (start 70.431 57.397999) (mid 69.93 56.897) (end 69.428999 57.397999) (width 0.79) (layer "F.Cu") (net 2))
 (arc (start 56.402999 65.918032) (mid 56.788369 64.91309) (end 58.140763 64.43348) (width 0.79) (layer "F.Cu") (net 2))
 (arc (start 61.413 145.310688) (mid 60.911999 145.811688) (end 60.411 145.310688) (width 0.79) (layer "F.Cu") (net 2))
 (arc (start 97.485 153.498) (mid 96.984 153.999) (end 96.483 153.498) (width 0.79) (layer "F.Cu") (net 2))
 (arc (start 59.409 144.998705) (mid 58.907999 145.499705) (end 58.407 144.998705) (width 0.79) (layer "F.Cu") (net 2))
 (arc (start 92.475 57.397999) (mid 91.974 56.897) (end 91.473 57.397999) (width 0.79) (layer "F.Cu") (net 2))
 (arc (start 74.439 57.397999) (mid 73.937999 56.897) (end 73.437 57.397999) (width 0.79) (layer "F.Cu") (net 2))
 (arc (start 106.503 116.228749) (mid 105.876749 116.855) (end 105.2505 116.228749) (width 0.79) (layer "F.Cu") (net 2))
 (arc (start 96.483 62.896) (mid 95.982 62.394999) (end 95.481 62.896) (width 0.79) (layer "F.Cu") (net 2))
 (arc (start 103.496999 86.354) (mid 102.996 86.855) (end 102.494999 86.354) (width 0.79) (layer "F.Cu") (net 2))
 (arc (start 68.427 57.397999) (mid 67.926 56.897) (end 67.425 57.397999) (width 0.79) (layer "F.Cu") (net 2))
 (arc (start 60.411 65.944632) (mid 59.91 65.443632) (end 59.409 65.944632) (width 0.79) (layer "F.Cu") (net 2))
 (arc (start 102.494999 56.395999) (mid 101.993999 55.894999) (end 101.492999 56.395999) (width 0.79) (layer "F.Cu") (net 2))
 (arc (start 103.997999 116.228749) (mid 103.371749 116.855) (end 102.7455 116.228749) (width 0.79) (layer "F.Cu") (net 2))
 (arc (start 75.440999 153.498) (mid 74.94 153.999) (end 74.439 153.498) (width 0.79) (layer "F.Cu") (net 2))
 (arc (start 80.451 57.397999) (mid 79.949999 56.897) (end 79.449 57.397999) (width 0.79) (layer "F.Cu") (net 2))
 (arc (start 71.433 153.498) (mid 70.931999 153.999) (end 70.431 153.498) (width 0.79) (layer "F.Cu") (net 2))
 (arc (start 67.425 153.498) (mid 66.923999 153.999) (end 66.423 153.498) (width 0.79) (layer "F.Cu") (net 2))
 (arc (start 78.447 57.397999) (mid 77.946 56.897) (end 77.445 57.397999) (width 0.79) (layer "F.Cu") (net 2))
 (arc (start 77.445 153.498) (mid 76.944 153.999) (end 76.443 153.498) (width 0.79) (layer "F.Cu") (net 2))
 (arc (start 105.500999 86.354) (mid 105 86.855) (end 104.499 86.354) (width 0.79) (layer "F.Cu") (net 2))
 (arc (start 76.443 57.397999) (mid 75.942 56.897) (end 75.440999 57.397999) (width 0.79) (layer "F.Cu") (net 2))
 (arc (start 85.461 153.498) (mid 84.96 153.999) (end 84.458999 153.498) (width 0.79) (layer "F.Cu") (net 2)))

